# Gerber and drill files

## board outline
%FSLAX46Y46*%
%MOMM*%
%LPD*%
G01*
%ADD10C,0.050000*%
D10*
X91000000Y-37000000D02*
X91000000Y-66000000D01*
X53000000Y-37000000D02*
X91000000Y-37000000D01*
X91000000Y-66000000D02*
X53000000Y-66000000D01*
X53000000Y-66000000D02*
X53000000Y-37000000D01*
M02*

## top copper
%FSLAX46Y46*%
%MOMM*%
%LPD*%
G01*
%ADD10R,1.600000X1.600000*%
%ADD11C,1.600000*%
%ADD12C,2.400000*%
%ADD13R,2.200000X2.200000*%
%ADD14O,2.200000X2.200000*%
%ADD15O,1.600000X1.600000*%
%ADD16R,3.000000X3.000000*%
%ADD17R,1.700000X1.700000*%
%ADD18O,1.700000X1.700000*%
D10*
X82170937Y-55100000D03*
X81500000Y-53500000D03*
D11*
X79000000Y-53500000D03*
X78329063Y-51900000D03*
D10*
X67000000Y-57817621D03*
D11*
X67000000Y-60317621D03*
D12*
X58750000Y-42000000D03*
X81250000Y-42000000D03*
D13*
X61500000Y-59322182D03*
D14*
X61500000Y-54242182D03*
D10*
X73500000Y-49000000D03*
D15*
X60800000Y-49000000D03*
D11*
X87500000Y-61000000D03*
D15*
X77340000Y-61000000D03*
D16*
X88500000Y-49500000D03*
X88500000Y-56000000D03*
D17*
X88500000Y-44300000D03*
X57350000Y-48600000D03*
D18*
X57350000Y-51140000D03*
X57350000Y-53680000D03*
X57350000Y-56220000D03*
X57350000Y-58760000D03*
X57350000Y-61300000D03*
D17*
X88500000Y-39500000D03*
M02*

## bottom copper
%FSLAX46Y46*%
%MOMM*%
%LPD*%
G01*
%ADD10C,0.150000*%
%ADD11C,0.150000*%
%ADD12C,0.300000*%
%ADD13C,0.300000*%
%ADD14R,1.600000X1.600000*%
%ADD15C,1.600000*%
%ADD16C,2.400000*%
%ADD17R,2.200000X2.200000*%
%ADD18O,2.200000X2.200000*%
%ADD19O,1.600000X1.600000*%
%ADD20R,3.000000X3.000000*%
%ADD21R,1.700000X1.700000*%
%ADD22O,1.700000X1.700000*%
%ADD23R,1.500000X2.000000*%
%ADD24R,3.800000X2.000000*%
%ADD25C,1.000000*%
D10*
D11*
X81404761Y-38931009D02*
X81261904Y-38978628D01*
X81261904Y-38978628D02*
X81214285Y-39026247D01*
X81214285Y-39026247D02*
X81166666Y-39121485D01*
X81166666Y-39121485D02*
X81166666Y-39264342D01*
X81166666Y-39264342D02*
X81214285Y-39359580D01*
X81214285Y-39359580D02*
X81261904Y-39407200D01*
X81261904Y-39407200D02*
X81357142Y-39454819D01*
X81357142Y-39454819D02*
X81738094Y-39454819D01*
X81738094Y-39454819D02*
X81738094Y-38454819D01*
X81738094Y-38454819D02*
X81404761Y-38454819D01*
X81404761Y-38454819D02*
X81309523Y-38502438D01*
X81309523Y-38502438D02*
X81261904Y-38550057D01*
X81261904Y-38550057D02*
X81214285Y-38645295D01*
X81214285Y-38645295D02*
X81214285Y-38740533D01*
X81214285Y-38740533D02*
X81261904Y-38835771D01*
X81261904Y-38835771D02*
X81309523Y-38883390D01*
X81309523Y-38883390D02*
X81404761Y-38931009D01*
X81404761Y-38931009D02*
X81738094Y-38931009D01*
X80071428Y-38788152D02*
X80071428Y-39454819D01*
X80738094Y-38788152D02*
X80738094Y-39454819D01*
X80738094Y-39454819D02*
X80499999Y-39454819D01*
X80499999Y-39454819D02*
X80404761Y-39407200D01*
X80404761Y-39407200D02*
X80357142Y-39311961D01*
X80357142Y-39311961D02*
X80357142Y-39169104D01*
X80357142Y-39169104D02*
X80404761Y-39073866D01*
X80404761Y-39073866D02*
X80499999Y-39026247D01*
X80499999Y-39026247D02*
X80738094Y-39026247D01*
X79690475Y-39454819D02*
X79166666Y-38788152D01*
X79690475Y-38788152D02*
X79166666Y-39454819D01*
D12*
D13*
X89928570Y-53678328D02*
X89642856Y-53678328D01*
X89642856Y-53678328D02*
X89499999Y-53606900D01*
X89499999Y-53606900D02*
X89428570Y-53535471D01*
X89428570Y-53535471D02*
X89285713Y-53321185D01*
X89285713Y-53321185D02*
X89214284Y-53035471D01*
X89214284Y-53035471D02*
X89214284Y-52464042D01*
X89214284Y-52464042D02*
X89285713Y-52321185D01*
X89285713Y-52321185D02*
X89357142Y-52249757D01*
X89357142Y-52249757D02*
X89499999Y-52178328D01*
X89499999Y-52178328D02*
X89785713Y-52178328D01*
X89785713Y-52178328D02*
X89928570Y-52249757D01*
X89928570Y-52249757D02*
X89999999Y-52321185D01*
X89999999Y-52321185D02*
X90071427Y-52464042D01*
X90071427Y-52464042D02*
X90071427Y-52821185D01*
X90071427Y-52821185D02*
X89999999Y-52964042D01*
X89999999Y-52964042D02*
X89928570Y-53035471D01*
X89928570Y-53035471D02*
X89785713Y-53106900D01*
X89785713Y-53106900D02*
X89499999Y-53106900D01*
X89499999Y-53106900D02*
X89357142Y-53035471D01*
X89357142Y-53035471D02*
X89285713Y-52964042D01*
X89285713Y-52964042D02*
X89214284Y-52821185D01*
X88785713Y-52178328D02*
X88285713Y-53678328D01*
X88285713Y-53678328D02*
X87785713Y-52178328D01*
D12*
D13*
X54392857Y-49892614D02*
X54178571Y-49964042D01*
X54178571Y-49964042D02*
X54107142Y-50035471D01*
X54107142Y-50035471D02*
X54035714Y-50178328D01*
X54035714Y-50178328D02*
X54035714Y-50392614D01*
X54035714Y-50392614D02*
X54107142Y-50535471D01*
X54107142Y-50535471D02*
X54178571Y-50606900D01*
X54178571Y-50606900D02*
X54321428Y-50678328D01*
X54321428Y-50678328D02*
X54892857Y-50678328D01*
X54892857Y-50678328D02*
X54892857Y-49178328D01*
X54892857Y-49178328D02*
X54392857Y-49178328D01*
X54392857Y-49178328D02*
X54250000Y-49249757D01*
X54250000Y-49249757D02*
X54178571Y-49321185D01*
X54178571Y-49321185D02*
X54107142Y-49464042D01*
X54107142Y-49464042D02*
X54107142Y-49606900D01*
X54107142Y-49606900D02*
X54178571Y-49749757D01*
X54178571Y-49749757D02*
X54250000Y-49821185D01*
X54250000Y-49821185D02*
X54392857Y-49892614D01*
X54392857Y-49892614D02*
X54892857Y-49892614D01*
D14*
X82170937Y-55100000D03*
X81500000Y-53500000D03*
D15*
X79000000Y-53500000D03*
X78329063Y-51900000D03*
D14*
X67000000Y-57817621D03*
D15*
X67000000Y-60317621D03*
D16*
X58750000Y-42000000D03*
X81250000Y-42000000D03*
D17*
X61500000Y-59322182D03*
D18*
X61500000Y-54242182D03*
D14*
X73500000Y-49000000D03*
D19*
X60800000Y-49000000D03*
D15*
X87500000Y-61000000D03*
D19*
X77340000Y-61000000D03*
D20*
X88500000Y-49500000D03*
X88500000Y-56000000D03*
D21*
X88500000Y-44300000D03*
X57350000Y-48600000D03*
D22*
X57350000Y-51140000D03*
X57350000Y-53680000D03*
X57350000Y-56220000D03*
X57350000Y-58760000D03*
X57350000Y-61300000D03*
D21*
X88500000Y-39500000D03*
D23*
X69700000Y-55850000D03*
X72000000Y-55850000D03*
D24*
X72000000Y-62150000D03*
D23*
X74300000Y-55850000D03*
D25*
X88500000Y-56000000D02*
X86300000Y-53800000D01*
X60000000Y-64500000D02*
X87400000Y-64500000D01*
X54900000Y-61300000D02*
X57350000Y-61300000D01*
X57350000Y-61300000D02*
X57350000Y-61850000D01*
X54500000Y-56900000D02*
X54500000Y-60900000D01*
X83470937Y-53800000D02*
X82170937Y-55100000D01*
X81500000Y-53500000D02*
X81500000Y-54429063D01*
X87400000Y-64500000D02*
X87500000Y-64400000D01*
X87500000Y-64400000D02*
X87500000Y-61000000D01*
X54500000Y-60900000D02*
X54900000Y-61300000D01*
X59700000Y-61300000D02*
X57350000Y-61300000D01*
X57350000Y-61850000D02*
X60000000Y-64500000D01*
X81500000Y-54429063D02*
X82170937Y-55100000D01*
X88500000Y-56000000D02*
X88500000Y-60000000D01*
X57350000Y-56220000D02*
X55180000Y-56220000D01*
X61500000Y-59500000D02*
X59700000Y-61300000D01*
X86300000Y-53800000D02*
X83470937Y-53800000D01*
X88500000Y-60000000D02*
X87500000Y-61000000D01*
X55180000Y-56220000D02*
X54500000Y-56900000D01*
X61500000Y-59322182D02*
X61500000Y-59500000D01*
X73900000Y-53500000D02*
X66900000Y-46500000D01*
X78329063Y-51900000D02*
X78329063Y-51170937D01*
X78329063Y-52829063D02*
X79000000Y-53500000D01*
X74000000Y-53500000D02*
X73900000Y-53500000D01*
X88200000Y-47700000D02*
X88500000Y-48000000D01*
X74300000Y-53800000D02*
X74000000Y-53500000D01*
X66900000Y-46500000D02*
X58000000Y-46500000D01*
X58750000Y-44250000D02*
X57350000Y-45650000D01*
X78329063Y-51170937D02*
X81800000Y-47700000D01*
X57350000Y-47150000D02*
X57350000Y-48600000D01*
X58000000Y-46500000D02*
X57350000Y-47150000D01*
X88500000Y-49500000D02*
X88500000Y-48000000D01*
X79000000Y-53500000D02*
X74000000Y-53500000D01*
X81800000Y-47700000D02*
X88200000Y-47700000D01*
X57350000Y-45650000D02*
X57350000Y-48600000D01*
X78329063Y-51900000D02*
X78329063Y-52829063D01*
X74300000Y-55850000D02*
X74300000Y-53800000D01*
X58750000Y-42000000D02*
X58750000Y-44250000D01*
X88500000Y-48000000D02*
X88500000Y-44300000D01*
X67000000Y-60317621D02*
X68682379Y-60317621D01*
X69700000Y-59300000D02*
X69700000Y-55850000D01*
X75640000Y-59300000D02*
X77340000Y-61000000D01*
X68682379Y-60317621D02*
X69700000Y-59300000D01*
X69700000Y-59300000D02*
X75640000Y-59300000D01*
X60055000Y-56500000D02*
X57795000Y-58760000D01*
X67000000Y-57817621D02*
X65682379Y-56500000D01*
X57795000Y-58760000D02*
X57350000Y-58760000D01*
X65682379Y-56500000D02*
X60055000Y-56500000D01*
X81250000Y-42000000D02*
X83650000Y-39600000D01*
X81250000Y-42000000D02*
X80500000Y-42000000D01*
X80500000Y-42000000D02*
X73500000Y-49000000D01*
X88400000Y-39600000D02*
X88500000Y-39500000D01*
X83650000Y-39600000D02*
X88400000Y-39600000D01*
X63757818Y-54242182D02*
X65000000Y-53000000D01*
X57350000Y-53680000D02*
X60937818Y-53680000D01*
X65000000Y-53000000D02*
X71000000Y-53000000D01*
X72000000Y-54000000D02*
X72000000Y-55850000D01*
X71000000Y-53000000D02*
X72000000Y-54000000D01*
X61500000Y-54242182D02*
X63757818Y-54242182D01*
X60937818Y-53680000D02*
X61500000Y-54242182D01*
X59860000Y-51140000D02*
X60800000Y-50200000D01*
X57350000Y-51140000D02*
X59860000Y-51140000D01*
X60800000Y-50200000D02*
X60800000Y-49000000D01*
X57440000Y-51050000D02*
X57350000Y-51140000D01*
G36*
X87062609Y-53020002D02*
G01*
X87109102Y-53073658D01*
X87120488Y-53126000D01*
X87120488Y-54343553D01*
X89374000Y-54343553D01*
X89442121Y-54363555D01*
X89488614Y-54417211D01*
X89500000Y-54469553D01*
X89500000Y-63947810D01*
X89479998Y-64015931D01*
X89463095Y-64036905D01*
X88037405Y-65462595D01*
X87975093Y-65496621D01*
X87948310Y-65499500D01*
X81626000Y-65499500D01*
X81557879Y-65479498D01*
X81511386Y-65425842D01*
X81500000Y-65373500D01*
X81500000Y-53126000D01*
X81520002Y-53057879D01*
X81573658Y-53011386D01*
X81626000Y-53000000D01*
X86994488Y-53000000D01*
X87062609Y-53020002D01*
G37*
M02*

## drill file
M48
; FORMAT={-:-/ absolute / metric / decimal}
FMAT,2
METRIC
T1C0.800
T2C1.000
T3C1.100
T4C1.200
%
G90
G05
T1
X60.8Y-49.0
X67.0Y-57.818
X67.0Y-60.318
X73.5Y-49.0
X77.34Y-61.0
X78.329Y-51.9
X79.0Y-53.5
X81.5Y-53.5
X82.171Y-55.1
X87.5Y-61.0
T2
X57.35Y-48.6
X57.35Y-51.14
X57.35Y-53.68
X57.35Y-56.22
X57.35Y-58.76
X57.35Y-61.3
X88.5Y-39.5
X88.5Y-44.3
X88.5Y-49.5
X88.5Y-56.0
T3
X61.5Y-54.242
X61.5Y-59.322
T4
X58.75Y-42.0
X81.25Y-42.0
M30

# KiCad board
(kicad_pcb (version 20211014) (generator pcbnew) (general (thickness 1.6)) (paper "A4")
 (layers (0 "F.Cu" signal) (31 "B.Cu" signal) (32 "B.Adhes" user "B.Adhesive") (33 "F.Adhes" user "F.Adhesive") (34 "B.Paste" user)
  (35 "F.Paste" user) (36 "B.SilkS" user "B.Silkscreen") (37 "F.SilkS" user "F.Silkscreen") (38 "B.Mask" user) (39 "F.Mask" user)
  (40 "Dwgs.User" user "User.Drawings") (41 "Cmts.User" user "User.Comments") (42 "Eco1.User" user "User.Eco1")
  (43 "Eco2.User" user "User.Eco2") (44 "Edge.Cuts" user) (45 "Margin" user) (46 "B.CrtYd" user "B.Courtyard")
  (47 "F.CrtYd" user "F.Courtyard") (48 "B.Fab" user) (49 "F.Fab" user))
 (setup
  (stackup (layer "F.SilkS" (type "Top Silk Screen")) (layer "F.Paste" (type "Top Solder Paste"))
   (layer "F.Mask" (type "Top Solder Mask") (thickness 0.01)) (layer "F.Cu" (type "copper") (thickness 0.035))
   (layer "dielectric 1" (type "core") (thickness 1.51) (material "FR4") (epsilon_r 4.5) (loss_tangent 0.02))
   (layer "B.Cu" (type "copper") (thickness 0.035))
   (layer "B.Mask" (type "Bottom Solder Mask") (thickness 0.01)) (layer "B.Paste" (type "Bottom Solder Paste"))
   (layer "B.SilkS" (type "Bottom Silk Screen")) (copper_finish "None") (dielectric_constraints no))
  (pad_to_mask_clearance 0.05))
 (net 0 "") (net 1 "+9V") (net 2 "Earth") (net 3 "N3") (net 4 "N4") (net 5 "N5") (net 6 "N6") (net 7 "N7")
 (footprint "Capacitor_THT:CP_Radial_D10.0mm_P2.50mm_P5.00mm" (layer "F.Cu") (at 81.5 53.5 180)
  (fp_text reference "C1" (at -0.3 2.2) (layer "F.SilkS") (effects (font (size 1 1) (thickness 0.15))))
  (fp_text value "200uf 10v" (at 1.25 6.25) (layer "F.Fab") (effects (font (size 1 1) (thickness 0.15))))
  (pad "1" thru_hole rect locked (at -0.670937 -1.6 180) (size 1.6 1.6) (drill 0.8) (layers *.Cu *.Mask) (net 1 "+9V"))
  (pad "1" thru_hole rect locked (at 0 0 180) (size 1.6 1.6) (drill 0.8) (layers *.Cu *.Mask) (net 1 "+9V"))
  (pad "2" thru_hole circle locked (at 2.5 0 180) (size 1.6 1.6) (drill 0.8) (layers *.Cu *.Mask) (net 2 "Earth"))
  (pad "2" thru_hole circle locked (at 3.170937 1.6 180) (size 1.6 1.6) (drill 0.8) (layers *.Cu *.Mask) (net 2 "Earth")))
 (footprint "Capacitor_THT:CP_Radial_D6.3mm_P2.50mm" (layer "F.Cu") (at 67 57.817621 -90)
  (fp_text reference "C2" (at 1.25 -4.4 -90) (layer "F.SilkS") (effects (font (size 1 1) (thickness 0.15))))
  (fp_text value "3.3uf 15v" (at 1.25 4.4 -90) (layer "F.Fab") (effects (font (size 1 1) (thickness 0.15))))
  (pad "1" thru_hole rect locked (at 0 0 270) (size 1.6 1.6) (drill 0.8) (layers *.Cu *.Mask) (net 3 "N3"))
  (pad "2" thru_hole circle locked (at 2.5 0 270) (size 1.6 1.6) (drill 0.8) (layers *.Cu *.Mask) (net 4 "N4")))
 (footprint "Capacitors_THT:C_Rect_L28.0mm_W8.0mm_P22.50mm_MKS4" (layer "F.Cu") (at 58.75 42)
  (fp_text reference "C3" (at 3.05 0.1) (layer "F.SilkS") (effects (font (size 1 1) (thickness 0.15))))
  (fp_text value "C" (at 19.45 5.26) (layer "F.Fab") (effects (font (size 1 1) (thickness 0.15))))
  (pad "1" thru_hole circle locked (at 0 0) (size 2.4 2.4) (drill 1.2) (layers *.Cu *.Mask) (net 2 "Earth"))
  (pad "2" thru_hole circle locked (at 22.5 0) (size 2.4 2.4) (drill 1.2) (layers *.Cu *.Mask) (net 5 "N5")))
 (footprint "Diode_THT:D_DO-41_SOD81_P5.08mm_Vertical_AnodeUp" (layer "F.Cu") (at 61.5 59.322182 90)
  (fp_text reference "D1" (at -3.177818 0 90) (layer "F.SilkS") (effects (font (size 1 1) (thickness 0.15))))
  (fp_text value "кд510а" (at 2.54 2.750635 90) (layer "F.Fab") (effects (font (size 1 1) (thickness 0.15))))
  (pad "1" thru_hole rect locked (at 0 0 90) (size 2.2 2.2) (drill 1.1) (layers *.Cu *.Mask) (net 1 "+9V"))
  (pad "2" thru_hole oval locked (at 5.08 0 90) (size 2.2 2.2) (drill 1.1) (layers *.Cu *.Mask) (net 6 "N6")))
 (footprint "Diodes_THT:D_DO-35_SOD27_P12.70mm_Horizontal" (layer "F.Cu") (at 73.5 49 180)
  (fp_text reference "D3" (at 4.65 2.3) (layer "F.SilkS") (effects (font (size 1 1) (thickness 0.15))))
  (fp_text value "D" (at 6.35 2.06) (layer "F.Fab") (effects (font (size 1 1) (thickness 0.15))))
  (pad "1" thru_hole rect locked (at 0 0 180) (size 1.6 1.6) (drill 0.8) (layers *.Cu *.Mask) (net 5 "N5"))
  (pad "2" thru_hole oval locked (at 12.7 0 180) (size 1.6 1.6) (drill 0.8) (layers *.Cu *.Mask) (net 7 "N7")))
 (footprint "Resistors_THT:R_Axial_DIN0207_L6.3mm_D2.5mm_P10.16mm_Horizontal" (layer "F.Cu") (at 87.5 61 180)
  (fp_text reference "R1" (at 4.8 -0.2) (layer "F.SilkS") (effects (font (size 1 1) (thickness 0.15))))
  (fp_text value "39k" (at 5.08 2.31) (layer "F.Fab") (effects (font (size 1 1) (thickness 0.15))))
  (pad "1" thru_hole circle locked (at 0 0 180) (size 1.6 1.6) (drill 0.8) (layers *.Cu *.Mask) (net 1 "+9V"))
  (pad "2" thru_hole oval locked (at 10.16 0 180) (size 1.6 1.6) (drill 0.8) (layers *.Cu *.Mask) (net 4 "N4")))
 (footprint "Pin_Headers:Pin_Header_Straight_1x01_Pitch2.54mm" (layer "F.Cu") (at 88.5 49.5 90)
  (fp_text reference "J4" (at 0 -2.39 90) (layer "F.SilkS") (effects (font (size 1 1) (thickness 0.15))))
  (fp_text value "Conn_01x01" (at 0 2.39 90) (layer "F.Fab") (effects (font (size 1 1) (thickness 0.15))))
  (pad "1" thru_hole rect locked (at 0 0 90) (size 3 3) (drill 1) (layers *.Cu *.Mask) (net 2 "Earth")))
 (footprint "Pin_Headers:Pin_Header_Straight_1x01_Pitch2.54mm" (layer "F.Cu") (at 88.5 56 90)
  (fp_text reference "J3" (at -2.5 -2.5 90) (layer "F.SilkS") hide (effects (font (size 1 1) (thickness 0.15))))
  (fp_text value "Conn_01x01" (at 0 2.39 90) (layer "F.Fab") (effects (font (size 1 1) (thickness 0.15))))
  (pad "1" thru_hole rect locked (at 0 0 90) (size 3 3) (drill 1) (layers *.Cu *.Mask) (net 1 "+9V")))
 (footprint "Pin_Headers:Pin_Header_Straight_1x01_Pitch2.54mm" (layer "F.Cu") (at 88.5 44.3)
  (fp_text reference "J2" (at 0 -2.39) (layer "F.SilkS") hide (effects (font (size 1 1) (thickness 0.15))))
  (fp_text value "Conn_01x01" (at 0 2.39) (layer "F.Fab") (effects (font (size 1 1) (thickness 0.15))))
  (pad "1" thru_hole rect locked (at 0 0) (size 1.7 1.7) (drill 1) (layers *.Cu *.Mask) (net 2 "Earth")))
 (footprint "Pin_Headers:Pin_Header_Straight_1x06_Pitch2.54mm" (layer "F.Cu") (at 57.35 48.6)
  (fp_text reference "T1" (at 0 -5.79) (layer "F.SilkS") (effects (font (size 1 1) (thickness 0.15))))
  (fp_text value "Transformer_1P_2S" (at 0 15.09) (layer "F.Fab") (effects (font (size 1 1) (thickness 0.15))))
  (pad "1" thru_hole rect locked (at 0 0) (size 1.7 1.7) (drill 1) (layers *.Cu *.Mask) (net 2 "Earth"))
  (pad "2" thru_hole oval locked (at 0 2.54) (size 1.7 1.7) (drill 1) (layers *.Cu *.Mask) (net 7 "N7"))
  (pad "3" thru_hole oval locked (at 0 5.08) (size 1.7 1.7) (drill 1) (layers *.Cu *.Mask) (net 6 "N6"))
  (pad "4" thru_hole oval locked (at 0 7.62) (size 1.7 1.7) (drill 1) (layers *.Cu *.Mask) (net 1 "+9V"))
  (pad "5" thru_hole oval locked (at 0 10.16) (size 1.7 1.7) (drill 1) (layers *.Cu *.Mask) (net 3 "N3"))
  (pad "6" thru_hole oval locked (at 0 12.7) (size 1.7 1.7) (drill 1) (layers *.Cu *.Mask) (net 1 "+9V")))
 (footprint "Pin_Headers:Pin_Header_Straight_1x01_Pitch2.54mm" (layer "F.Cu") (at 88.5 39.5)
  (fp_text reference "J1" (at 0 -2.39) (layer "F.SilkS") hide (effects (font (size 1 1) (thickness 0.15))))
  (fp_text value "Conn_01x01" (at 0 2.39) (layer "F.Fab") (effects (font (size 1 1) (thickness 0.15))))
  (pad "1" thru_hole rect locked (at 0 0) (size 1.7 1.7) (drill 1) (layers *.Cu *.Mask) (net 5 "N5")))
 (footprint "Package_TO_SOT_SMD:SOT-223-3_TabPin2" (layer "B.Cu") (at 72 59 -90)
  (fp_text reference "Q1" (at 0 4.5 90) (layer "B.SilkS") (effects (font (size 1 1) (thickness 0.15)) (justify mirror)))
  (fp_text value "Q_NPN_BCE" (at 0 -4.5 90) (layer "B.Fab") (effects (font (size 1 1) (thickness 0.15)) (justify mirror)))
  (pad "1" smd rect locked (at -3.15 2.3 270) (size 2 1.5) (layers "B.Cu" "B.Paste" "B.Mask") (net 4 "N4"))
  (pad "2" smd rect locked (at -3.15 0 270) (size 2 1.5) (layers "B.Cu" "B.Paste" "B.Mask") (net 6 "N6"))
  (pad "2" smd rect locked (at 3.15 0 270) (size 2 3.8) (layers "B.Cu" "B.Paste" "B.Mask") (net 6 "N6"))
  (pad "3" smd rect locked (at -3.15 -2.3 270) (size 2 1.5) (layers "B.Cu" "B.Paste" "B.Mask") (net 2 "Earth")))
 (gr_line (start 91 37) (end 91 66) (layer "Edge.Cuts") (width 0.05))
 (gr_line (start 53 37) (end 91 37) (layer "Edge.Cuts") (width 0.05))
 (gr_line (start 91 66) (end 53 66) (layer "Edge.Cuts") (width 0.05))
 (gr_line (start 53 66) (end 53 37) (layer "Edge.Cuts") (width 0.05))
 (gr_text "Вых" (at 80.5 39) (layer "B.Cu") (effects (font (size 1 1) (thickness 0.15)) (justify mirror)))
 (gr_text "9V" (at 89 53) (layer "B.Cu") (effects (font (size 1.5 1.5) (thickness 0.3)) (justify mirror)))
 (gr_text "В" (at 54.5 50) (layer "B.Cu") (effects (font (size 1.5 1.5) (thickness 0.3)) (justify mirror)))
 (segment (start 88.5 56) (end 86.3 53.8) (width 1) (layer "B.Cu") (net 1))
 (segment (start 60 64.5) (end 87.4 64.5) (width 1) (layer "B.Cu") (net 1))
 (segment (start 54.9 61.3) (end 57.35 61.3) (width 1) (layer "B.Cu") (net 1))
 (segment (start 57.35 61.3) (end 57.35 61.85) (width 1) (layer "B.Cu") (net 1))
 (segment (start 54.5 56.9) (end 54.5 60.9) (width 1) (layer "B.Cu") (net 1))
 (segment (start 83.470937 53.8) (end 82.170937 55.1) (width 1) (layer "B.Cu") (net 1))
 (segment (start 81.5 53.5) (end 81.5 54.429063) (width 1) (layer "B.Cu") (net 1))
 (segment (start 87.4 64.5) (end 87.5 64.4) (width 1) (layer "B.Cu") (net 1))
 (segment (start 87.5 64.4) (end 87.5 61) (width 1) (layer "B.Cu") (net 1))
 (segment (start 54.5 60.9) (end 54.9 61.3) (width 1) (layer "B.Cu") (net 1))
 (segment (start 59.7 61.3) (end 57.35 61.3) (width 1) (layer "B.Cu") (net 1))
 (segment (start 57.35 61.85) (end 60 64.5) (width 1) (layer "B.Cu") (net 1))
 (segment (start 81.5 54.429063) (end 82.170937 55.1) (width 1) (layer "B.Cu") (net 1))
 (segment (start 88.5 56) (end 88.5 60) (width 1) (layer "B.Cu") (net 1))
 (segment (start 57.35 56.22) (end 55.18 56.22) (width 1) (layer "B.Cu") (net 1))
 (segment (start 61.5 59.5) (end 59.7 61.3) (width 1) (layer "B.Cu") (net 1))
 (segment (start 86.3 53.8) (end 83.470937 53.8) (width 1) (layer "B.Cu") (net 1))
 (segment (start 88.5 60) (end 87.5 61) (width 1) (layer "B.Cu") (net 1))
 (segment (start 55.18 56.22) (end 54.5 56.9) (width 1) (layer "B.Cu") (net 1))
 (segment (start 61.5 59.322182) (end 61.5 59.5) (width 1) (layer "B.Cu") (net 1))
 (segment (start 73.9 53.5) (end 66.9 46.5) (width 1) (layer "B.Cu") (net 2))
 (segment (start 78.329063 51.9) (end 78.329063 51.170937) (width 1) (layer "B.Cu") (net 2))
 (segment (start 78.329063 52.829063) (end 79 53.5) (width 1) (layer "B.Cu") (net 2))
 (segment (start 74 53.5) (end 73.9 53.5) (width 1) (layer "B.Cu") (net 2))
 (segment (start 88.2 47.7) (end 88.5 48) (width 1) (layer "B.Cu") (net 2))
 (segment (start 74.3 53.8) (end 74 53.5) (width 1) (layer "B.Cu") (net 2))
 (segment (start 66.9 46.5) (end 58 46.5) (width 1) (layer "B.Cu") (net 2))
 (segment (start 58.75 44.25) (end 57.35 45.65) (width 1) (layer "B.Cu") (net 2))
 (segment (start 78.329063 51.170937) (end 81.8 47.7) (width 1) (layer "B.Cu") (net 2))
 (segment (start 57.35 47.15) (end 57.35 48.6) (width 1) (layer "B.Cu") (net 2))
 (segment (start 58 46.5) (end 57.35 47.15) (width 1) (layer "B.Cu") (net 2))
 (segment (start 88.5 49.5) (end 88.5 48) (width 1) (layer "B.Cu") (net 2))
 (segment (start 79 53.5) (end 74 53.5) (width 1) (layer "B.Cu") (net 2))
 (segment (start 81.8 47.7) (end 88.2 47.7) (width 1) (layer "B.Cu") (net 2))
 (segment (start 57.35 45.65) (end 57.35 48.6) (width 1) (layer "B.Cu") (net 2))
 (segment (start 78.329063 51.9) (end 78.329063 52.829063) (width 1) (layer "B.Cu") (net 2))
 (segment (start 74.3 55.85) (end 74.3 53.8) (width 1) (layer "B.Cu") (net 2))
 (segment (start 58.75 42) (end 58.75 44.25) (width 1) (layer "B.Cu") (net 2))
 (segment (start 88.5 48) (end 88.5 44.3) (width 1) (layer "B.Cu") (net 2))
 (segment (start 67 60.317621) (end 68.682379 60.317621) (width 1) (layer "B.Cu") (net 4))
 (segment (start 69.7 59.3) (end 69.7 55.85) (width 1) (layer "B.Cu") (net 4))
 (segment (start 75.64 59.3) (end 77.34 61) (width 1) (layer "B.Cu") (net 4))
 (segment (start 68.682379 60.317621) (end 69.7 59.3) (width 1) (layer "B.Cu") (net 4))
 (segment (start 69.7 59.3) (end 75.64 59.3) (width 1) (layer "B.Cu") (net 4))
 (segment (start 60.055 56.5) (end 57.795 58.76) (width 1) (layer "B.Cu") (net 3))
 (segment (start 67 57.817621) (end 65.682379 56.5) (width 1) (layer "B.Cu") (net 3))
 (segment (start 57.795 58.76) (end 57.35 58.76) (width 1) (layer "B.Cu") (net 3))
 (segment (start 65.682379 56.5) (end 60.055 56.5) (width 1) (layer "B.Cu") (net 3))
 (segment (start 81.25 42) (end 83.65 39.6) (width 1) (layer "B.Cu") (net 5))
 (segment (start 81.25 42) (end 80.5 42) (width 1) (layer "B.Cu") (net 5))
 (segment (start 80.5 42) (end 73.5 49) (width 1) (layer "B.Cu") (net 5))
 (segment (start 88.4 39.6) (end 88.5 39.5) (width 1) (layer "B.Cu") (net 5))
 (segment (start 83.65 39.6) (end 88.4 39.6) (width 1) (layer "B.Cu") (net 5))
 (segment (start 63.757818 54.242182) (end 65 53) (width 1) (layer "B.Cu") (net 6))
 (segment (start 57.35 53.68) (end 60.937818 53.68) (width 1) (layer "B.Cu") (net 6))
 (segment (start 65 53) (end 71 53) (width 1) (layer "B.Cu") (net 6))
 (segment (start 72 54) (end 72 55.85) (width 1) (layer "B.Cu") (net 6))
 (segment (start 71 53) (end 72 54) (width 1) (layer "B.Cu") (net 6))
 (segment (start 61.5 54.242182) (end 63.757818 54.242182) (width 1) (layer "B.Cu") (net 6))
 (segment (start 60.937818 53.68) (end 61.5 54.242182) (width 1) (layer "B.Cu") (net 6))
 (segment (start 59.86 51.14) (end 60.8 50.2) (width 1) (layer "B.Cu") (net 7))
 (segment (start 57.35 51.14) (end 59.86 51.14) (width 1) (layer "B.Cu") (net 7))
 (segment (start 60.8 50.2) (end 60.8 49) (width 1) (layer "B.Cu") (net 7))
 (segment (start 57.44 51.05) (end 57.35 51.14) (width 1) (layer "B.Cu") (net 7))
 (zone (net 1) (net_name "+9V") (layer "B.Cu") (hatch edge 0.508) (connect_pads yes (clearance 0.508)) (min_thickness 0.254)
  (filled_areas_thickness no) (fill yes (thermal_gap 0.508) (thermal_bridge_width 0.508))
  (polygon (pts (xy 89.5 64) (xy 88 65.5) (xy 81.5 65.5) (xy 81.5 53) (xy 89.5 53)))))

